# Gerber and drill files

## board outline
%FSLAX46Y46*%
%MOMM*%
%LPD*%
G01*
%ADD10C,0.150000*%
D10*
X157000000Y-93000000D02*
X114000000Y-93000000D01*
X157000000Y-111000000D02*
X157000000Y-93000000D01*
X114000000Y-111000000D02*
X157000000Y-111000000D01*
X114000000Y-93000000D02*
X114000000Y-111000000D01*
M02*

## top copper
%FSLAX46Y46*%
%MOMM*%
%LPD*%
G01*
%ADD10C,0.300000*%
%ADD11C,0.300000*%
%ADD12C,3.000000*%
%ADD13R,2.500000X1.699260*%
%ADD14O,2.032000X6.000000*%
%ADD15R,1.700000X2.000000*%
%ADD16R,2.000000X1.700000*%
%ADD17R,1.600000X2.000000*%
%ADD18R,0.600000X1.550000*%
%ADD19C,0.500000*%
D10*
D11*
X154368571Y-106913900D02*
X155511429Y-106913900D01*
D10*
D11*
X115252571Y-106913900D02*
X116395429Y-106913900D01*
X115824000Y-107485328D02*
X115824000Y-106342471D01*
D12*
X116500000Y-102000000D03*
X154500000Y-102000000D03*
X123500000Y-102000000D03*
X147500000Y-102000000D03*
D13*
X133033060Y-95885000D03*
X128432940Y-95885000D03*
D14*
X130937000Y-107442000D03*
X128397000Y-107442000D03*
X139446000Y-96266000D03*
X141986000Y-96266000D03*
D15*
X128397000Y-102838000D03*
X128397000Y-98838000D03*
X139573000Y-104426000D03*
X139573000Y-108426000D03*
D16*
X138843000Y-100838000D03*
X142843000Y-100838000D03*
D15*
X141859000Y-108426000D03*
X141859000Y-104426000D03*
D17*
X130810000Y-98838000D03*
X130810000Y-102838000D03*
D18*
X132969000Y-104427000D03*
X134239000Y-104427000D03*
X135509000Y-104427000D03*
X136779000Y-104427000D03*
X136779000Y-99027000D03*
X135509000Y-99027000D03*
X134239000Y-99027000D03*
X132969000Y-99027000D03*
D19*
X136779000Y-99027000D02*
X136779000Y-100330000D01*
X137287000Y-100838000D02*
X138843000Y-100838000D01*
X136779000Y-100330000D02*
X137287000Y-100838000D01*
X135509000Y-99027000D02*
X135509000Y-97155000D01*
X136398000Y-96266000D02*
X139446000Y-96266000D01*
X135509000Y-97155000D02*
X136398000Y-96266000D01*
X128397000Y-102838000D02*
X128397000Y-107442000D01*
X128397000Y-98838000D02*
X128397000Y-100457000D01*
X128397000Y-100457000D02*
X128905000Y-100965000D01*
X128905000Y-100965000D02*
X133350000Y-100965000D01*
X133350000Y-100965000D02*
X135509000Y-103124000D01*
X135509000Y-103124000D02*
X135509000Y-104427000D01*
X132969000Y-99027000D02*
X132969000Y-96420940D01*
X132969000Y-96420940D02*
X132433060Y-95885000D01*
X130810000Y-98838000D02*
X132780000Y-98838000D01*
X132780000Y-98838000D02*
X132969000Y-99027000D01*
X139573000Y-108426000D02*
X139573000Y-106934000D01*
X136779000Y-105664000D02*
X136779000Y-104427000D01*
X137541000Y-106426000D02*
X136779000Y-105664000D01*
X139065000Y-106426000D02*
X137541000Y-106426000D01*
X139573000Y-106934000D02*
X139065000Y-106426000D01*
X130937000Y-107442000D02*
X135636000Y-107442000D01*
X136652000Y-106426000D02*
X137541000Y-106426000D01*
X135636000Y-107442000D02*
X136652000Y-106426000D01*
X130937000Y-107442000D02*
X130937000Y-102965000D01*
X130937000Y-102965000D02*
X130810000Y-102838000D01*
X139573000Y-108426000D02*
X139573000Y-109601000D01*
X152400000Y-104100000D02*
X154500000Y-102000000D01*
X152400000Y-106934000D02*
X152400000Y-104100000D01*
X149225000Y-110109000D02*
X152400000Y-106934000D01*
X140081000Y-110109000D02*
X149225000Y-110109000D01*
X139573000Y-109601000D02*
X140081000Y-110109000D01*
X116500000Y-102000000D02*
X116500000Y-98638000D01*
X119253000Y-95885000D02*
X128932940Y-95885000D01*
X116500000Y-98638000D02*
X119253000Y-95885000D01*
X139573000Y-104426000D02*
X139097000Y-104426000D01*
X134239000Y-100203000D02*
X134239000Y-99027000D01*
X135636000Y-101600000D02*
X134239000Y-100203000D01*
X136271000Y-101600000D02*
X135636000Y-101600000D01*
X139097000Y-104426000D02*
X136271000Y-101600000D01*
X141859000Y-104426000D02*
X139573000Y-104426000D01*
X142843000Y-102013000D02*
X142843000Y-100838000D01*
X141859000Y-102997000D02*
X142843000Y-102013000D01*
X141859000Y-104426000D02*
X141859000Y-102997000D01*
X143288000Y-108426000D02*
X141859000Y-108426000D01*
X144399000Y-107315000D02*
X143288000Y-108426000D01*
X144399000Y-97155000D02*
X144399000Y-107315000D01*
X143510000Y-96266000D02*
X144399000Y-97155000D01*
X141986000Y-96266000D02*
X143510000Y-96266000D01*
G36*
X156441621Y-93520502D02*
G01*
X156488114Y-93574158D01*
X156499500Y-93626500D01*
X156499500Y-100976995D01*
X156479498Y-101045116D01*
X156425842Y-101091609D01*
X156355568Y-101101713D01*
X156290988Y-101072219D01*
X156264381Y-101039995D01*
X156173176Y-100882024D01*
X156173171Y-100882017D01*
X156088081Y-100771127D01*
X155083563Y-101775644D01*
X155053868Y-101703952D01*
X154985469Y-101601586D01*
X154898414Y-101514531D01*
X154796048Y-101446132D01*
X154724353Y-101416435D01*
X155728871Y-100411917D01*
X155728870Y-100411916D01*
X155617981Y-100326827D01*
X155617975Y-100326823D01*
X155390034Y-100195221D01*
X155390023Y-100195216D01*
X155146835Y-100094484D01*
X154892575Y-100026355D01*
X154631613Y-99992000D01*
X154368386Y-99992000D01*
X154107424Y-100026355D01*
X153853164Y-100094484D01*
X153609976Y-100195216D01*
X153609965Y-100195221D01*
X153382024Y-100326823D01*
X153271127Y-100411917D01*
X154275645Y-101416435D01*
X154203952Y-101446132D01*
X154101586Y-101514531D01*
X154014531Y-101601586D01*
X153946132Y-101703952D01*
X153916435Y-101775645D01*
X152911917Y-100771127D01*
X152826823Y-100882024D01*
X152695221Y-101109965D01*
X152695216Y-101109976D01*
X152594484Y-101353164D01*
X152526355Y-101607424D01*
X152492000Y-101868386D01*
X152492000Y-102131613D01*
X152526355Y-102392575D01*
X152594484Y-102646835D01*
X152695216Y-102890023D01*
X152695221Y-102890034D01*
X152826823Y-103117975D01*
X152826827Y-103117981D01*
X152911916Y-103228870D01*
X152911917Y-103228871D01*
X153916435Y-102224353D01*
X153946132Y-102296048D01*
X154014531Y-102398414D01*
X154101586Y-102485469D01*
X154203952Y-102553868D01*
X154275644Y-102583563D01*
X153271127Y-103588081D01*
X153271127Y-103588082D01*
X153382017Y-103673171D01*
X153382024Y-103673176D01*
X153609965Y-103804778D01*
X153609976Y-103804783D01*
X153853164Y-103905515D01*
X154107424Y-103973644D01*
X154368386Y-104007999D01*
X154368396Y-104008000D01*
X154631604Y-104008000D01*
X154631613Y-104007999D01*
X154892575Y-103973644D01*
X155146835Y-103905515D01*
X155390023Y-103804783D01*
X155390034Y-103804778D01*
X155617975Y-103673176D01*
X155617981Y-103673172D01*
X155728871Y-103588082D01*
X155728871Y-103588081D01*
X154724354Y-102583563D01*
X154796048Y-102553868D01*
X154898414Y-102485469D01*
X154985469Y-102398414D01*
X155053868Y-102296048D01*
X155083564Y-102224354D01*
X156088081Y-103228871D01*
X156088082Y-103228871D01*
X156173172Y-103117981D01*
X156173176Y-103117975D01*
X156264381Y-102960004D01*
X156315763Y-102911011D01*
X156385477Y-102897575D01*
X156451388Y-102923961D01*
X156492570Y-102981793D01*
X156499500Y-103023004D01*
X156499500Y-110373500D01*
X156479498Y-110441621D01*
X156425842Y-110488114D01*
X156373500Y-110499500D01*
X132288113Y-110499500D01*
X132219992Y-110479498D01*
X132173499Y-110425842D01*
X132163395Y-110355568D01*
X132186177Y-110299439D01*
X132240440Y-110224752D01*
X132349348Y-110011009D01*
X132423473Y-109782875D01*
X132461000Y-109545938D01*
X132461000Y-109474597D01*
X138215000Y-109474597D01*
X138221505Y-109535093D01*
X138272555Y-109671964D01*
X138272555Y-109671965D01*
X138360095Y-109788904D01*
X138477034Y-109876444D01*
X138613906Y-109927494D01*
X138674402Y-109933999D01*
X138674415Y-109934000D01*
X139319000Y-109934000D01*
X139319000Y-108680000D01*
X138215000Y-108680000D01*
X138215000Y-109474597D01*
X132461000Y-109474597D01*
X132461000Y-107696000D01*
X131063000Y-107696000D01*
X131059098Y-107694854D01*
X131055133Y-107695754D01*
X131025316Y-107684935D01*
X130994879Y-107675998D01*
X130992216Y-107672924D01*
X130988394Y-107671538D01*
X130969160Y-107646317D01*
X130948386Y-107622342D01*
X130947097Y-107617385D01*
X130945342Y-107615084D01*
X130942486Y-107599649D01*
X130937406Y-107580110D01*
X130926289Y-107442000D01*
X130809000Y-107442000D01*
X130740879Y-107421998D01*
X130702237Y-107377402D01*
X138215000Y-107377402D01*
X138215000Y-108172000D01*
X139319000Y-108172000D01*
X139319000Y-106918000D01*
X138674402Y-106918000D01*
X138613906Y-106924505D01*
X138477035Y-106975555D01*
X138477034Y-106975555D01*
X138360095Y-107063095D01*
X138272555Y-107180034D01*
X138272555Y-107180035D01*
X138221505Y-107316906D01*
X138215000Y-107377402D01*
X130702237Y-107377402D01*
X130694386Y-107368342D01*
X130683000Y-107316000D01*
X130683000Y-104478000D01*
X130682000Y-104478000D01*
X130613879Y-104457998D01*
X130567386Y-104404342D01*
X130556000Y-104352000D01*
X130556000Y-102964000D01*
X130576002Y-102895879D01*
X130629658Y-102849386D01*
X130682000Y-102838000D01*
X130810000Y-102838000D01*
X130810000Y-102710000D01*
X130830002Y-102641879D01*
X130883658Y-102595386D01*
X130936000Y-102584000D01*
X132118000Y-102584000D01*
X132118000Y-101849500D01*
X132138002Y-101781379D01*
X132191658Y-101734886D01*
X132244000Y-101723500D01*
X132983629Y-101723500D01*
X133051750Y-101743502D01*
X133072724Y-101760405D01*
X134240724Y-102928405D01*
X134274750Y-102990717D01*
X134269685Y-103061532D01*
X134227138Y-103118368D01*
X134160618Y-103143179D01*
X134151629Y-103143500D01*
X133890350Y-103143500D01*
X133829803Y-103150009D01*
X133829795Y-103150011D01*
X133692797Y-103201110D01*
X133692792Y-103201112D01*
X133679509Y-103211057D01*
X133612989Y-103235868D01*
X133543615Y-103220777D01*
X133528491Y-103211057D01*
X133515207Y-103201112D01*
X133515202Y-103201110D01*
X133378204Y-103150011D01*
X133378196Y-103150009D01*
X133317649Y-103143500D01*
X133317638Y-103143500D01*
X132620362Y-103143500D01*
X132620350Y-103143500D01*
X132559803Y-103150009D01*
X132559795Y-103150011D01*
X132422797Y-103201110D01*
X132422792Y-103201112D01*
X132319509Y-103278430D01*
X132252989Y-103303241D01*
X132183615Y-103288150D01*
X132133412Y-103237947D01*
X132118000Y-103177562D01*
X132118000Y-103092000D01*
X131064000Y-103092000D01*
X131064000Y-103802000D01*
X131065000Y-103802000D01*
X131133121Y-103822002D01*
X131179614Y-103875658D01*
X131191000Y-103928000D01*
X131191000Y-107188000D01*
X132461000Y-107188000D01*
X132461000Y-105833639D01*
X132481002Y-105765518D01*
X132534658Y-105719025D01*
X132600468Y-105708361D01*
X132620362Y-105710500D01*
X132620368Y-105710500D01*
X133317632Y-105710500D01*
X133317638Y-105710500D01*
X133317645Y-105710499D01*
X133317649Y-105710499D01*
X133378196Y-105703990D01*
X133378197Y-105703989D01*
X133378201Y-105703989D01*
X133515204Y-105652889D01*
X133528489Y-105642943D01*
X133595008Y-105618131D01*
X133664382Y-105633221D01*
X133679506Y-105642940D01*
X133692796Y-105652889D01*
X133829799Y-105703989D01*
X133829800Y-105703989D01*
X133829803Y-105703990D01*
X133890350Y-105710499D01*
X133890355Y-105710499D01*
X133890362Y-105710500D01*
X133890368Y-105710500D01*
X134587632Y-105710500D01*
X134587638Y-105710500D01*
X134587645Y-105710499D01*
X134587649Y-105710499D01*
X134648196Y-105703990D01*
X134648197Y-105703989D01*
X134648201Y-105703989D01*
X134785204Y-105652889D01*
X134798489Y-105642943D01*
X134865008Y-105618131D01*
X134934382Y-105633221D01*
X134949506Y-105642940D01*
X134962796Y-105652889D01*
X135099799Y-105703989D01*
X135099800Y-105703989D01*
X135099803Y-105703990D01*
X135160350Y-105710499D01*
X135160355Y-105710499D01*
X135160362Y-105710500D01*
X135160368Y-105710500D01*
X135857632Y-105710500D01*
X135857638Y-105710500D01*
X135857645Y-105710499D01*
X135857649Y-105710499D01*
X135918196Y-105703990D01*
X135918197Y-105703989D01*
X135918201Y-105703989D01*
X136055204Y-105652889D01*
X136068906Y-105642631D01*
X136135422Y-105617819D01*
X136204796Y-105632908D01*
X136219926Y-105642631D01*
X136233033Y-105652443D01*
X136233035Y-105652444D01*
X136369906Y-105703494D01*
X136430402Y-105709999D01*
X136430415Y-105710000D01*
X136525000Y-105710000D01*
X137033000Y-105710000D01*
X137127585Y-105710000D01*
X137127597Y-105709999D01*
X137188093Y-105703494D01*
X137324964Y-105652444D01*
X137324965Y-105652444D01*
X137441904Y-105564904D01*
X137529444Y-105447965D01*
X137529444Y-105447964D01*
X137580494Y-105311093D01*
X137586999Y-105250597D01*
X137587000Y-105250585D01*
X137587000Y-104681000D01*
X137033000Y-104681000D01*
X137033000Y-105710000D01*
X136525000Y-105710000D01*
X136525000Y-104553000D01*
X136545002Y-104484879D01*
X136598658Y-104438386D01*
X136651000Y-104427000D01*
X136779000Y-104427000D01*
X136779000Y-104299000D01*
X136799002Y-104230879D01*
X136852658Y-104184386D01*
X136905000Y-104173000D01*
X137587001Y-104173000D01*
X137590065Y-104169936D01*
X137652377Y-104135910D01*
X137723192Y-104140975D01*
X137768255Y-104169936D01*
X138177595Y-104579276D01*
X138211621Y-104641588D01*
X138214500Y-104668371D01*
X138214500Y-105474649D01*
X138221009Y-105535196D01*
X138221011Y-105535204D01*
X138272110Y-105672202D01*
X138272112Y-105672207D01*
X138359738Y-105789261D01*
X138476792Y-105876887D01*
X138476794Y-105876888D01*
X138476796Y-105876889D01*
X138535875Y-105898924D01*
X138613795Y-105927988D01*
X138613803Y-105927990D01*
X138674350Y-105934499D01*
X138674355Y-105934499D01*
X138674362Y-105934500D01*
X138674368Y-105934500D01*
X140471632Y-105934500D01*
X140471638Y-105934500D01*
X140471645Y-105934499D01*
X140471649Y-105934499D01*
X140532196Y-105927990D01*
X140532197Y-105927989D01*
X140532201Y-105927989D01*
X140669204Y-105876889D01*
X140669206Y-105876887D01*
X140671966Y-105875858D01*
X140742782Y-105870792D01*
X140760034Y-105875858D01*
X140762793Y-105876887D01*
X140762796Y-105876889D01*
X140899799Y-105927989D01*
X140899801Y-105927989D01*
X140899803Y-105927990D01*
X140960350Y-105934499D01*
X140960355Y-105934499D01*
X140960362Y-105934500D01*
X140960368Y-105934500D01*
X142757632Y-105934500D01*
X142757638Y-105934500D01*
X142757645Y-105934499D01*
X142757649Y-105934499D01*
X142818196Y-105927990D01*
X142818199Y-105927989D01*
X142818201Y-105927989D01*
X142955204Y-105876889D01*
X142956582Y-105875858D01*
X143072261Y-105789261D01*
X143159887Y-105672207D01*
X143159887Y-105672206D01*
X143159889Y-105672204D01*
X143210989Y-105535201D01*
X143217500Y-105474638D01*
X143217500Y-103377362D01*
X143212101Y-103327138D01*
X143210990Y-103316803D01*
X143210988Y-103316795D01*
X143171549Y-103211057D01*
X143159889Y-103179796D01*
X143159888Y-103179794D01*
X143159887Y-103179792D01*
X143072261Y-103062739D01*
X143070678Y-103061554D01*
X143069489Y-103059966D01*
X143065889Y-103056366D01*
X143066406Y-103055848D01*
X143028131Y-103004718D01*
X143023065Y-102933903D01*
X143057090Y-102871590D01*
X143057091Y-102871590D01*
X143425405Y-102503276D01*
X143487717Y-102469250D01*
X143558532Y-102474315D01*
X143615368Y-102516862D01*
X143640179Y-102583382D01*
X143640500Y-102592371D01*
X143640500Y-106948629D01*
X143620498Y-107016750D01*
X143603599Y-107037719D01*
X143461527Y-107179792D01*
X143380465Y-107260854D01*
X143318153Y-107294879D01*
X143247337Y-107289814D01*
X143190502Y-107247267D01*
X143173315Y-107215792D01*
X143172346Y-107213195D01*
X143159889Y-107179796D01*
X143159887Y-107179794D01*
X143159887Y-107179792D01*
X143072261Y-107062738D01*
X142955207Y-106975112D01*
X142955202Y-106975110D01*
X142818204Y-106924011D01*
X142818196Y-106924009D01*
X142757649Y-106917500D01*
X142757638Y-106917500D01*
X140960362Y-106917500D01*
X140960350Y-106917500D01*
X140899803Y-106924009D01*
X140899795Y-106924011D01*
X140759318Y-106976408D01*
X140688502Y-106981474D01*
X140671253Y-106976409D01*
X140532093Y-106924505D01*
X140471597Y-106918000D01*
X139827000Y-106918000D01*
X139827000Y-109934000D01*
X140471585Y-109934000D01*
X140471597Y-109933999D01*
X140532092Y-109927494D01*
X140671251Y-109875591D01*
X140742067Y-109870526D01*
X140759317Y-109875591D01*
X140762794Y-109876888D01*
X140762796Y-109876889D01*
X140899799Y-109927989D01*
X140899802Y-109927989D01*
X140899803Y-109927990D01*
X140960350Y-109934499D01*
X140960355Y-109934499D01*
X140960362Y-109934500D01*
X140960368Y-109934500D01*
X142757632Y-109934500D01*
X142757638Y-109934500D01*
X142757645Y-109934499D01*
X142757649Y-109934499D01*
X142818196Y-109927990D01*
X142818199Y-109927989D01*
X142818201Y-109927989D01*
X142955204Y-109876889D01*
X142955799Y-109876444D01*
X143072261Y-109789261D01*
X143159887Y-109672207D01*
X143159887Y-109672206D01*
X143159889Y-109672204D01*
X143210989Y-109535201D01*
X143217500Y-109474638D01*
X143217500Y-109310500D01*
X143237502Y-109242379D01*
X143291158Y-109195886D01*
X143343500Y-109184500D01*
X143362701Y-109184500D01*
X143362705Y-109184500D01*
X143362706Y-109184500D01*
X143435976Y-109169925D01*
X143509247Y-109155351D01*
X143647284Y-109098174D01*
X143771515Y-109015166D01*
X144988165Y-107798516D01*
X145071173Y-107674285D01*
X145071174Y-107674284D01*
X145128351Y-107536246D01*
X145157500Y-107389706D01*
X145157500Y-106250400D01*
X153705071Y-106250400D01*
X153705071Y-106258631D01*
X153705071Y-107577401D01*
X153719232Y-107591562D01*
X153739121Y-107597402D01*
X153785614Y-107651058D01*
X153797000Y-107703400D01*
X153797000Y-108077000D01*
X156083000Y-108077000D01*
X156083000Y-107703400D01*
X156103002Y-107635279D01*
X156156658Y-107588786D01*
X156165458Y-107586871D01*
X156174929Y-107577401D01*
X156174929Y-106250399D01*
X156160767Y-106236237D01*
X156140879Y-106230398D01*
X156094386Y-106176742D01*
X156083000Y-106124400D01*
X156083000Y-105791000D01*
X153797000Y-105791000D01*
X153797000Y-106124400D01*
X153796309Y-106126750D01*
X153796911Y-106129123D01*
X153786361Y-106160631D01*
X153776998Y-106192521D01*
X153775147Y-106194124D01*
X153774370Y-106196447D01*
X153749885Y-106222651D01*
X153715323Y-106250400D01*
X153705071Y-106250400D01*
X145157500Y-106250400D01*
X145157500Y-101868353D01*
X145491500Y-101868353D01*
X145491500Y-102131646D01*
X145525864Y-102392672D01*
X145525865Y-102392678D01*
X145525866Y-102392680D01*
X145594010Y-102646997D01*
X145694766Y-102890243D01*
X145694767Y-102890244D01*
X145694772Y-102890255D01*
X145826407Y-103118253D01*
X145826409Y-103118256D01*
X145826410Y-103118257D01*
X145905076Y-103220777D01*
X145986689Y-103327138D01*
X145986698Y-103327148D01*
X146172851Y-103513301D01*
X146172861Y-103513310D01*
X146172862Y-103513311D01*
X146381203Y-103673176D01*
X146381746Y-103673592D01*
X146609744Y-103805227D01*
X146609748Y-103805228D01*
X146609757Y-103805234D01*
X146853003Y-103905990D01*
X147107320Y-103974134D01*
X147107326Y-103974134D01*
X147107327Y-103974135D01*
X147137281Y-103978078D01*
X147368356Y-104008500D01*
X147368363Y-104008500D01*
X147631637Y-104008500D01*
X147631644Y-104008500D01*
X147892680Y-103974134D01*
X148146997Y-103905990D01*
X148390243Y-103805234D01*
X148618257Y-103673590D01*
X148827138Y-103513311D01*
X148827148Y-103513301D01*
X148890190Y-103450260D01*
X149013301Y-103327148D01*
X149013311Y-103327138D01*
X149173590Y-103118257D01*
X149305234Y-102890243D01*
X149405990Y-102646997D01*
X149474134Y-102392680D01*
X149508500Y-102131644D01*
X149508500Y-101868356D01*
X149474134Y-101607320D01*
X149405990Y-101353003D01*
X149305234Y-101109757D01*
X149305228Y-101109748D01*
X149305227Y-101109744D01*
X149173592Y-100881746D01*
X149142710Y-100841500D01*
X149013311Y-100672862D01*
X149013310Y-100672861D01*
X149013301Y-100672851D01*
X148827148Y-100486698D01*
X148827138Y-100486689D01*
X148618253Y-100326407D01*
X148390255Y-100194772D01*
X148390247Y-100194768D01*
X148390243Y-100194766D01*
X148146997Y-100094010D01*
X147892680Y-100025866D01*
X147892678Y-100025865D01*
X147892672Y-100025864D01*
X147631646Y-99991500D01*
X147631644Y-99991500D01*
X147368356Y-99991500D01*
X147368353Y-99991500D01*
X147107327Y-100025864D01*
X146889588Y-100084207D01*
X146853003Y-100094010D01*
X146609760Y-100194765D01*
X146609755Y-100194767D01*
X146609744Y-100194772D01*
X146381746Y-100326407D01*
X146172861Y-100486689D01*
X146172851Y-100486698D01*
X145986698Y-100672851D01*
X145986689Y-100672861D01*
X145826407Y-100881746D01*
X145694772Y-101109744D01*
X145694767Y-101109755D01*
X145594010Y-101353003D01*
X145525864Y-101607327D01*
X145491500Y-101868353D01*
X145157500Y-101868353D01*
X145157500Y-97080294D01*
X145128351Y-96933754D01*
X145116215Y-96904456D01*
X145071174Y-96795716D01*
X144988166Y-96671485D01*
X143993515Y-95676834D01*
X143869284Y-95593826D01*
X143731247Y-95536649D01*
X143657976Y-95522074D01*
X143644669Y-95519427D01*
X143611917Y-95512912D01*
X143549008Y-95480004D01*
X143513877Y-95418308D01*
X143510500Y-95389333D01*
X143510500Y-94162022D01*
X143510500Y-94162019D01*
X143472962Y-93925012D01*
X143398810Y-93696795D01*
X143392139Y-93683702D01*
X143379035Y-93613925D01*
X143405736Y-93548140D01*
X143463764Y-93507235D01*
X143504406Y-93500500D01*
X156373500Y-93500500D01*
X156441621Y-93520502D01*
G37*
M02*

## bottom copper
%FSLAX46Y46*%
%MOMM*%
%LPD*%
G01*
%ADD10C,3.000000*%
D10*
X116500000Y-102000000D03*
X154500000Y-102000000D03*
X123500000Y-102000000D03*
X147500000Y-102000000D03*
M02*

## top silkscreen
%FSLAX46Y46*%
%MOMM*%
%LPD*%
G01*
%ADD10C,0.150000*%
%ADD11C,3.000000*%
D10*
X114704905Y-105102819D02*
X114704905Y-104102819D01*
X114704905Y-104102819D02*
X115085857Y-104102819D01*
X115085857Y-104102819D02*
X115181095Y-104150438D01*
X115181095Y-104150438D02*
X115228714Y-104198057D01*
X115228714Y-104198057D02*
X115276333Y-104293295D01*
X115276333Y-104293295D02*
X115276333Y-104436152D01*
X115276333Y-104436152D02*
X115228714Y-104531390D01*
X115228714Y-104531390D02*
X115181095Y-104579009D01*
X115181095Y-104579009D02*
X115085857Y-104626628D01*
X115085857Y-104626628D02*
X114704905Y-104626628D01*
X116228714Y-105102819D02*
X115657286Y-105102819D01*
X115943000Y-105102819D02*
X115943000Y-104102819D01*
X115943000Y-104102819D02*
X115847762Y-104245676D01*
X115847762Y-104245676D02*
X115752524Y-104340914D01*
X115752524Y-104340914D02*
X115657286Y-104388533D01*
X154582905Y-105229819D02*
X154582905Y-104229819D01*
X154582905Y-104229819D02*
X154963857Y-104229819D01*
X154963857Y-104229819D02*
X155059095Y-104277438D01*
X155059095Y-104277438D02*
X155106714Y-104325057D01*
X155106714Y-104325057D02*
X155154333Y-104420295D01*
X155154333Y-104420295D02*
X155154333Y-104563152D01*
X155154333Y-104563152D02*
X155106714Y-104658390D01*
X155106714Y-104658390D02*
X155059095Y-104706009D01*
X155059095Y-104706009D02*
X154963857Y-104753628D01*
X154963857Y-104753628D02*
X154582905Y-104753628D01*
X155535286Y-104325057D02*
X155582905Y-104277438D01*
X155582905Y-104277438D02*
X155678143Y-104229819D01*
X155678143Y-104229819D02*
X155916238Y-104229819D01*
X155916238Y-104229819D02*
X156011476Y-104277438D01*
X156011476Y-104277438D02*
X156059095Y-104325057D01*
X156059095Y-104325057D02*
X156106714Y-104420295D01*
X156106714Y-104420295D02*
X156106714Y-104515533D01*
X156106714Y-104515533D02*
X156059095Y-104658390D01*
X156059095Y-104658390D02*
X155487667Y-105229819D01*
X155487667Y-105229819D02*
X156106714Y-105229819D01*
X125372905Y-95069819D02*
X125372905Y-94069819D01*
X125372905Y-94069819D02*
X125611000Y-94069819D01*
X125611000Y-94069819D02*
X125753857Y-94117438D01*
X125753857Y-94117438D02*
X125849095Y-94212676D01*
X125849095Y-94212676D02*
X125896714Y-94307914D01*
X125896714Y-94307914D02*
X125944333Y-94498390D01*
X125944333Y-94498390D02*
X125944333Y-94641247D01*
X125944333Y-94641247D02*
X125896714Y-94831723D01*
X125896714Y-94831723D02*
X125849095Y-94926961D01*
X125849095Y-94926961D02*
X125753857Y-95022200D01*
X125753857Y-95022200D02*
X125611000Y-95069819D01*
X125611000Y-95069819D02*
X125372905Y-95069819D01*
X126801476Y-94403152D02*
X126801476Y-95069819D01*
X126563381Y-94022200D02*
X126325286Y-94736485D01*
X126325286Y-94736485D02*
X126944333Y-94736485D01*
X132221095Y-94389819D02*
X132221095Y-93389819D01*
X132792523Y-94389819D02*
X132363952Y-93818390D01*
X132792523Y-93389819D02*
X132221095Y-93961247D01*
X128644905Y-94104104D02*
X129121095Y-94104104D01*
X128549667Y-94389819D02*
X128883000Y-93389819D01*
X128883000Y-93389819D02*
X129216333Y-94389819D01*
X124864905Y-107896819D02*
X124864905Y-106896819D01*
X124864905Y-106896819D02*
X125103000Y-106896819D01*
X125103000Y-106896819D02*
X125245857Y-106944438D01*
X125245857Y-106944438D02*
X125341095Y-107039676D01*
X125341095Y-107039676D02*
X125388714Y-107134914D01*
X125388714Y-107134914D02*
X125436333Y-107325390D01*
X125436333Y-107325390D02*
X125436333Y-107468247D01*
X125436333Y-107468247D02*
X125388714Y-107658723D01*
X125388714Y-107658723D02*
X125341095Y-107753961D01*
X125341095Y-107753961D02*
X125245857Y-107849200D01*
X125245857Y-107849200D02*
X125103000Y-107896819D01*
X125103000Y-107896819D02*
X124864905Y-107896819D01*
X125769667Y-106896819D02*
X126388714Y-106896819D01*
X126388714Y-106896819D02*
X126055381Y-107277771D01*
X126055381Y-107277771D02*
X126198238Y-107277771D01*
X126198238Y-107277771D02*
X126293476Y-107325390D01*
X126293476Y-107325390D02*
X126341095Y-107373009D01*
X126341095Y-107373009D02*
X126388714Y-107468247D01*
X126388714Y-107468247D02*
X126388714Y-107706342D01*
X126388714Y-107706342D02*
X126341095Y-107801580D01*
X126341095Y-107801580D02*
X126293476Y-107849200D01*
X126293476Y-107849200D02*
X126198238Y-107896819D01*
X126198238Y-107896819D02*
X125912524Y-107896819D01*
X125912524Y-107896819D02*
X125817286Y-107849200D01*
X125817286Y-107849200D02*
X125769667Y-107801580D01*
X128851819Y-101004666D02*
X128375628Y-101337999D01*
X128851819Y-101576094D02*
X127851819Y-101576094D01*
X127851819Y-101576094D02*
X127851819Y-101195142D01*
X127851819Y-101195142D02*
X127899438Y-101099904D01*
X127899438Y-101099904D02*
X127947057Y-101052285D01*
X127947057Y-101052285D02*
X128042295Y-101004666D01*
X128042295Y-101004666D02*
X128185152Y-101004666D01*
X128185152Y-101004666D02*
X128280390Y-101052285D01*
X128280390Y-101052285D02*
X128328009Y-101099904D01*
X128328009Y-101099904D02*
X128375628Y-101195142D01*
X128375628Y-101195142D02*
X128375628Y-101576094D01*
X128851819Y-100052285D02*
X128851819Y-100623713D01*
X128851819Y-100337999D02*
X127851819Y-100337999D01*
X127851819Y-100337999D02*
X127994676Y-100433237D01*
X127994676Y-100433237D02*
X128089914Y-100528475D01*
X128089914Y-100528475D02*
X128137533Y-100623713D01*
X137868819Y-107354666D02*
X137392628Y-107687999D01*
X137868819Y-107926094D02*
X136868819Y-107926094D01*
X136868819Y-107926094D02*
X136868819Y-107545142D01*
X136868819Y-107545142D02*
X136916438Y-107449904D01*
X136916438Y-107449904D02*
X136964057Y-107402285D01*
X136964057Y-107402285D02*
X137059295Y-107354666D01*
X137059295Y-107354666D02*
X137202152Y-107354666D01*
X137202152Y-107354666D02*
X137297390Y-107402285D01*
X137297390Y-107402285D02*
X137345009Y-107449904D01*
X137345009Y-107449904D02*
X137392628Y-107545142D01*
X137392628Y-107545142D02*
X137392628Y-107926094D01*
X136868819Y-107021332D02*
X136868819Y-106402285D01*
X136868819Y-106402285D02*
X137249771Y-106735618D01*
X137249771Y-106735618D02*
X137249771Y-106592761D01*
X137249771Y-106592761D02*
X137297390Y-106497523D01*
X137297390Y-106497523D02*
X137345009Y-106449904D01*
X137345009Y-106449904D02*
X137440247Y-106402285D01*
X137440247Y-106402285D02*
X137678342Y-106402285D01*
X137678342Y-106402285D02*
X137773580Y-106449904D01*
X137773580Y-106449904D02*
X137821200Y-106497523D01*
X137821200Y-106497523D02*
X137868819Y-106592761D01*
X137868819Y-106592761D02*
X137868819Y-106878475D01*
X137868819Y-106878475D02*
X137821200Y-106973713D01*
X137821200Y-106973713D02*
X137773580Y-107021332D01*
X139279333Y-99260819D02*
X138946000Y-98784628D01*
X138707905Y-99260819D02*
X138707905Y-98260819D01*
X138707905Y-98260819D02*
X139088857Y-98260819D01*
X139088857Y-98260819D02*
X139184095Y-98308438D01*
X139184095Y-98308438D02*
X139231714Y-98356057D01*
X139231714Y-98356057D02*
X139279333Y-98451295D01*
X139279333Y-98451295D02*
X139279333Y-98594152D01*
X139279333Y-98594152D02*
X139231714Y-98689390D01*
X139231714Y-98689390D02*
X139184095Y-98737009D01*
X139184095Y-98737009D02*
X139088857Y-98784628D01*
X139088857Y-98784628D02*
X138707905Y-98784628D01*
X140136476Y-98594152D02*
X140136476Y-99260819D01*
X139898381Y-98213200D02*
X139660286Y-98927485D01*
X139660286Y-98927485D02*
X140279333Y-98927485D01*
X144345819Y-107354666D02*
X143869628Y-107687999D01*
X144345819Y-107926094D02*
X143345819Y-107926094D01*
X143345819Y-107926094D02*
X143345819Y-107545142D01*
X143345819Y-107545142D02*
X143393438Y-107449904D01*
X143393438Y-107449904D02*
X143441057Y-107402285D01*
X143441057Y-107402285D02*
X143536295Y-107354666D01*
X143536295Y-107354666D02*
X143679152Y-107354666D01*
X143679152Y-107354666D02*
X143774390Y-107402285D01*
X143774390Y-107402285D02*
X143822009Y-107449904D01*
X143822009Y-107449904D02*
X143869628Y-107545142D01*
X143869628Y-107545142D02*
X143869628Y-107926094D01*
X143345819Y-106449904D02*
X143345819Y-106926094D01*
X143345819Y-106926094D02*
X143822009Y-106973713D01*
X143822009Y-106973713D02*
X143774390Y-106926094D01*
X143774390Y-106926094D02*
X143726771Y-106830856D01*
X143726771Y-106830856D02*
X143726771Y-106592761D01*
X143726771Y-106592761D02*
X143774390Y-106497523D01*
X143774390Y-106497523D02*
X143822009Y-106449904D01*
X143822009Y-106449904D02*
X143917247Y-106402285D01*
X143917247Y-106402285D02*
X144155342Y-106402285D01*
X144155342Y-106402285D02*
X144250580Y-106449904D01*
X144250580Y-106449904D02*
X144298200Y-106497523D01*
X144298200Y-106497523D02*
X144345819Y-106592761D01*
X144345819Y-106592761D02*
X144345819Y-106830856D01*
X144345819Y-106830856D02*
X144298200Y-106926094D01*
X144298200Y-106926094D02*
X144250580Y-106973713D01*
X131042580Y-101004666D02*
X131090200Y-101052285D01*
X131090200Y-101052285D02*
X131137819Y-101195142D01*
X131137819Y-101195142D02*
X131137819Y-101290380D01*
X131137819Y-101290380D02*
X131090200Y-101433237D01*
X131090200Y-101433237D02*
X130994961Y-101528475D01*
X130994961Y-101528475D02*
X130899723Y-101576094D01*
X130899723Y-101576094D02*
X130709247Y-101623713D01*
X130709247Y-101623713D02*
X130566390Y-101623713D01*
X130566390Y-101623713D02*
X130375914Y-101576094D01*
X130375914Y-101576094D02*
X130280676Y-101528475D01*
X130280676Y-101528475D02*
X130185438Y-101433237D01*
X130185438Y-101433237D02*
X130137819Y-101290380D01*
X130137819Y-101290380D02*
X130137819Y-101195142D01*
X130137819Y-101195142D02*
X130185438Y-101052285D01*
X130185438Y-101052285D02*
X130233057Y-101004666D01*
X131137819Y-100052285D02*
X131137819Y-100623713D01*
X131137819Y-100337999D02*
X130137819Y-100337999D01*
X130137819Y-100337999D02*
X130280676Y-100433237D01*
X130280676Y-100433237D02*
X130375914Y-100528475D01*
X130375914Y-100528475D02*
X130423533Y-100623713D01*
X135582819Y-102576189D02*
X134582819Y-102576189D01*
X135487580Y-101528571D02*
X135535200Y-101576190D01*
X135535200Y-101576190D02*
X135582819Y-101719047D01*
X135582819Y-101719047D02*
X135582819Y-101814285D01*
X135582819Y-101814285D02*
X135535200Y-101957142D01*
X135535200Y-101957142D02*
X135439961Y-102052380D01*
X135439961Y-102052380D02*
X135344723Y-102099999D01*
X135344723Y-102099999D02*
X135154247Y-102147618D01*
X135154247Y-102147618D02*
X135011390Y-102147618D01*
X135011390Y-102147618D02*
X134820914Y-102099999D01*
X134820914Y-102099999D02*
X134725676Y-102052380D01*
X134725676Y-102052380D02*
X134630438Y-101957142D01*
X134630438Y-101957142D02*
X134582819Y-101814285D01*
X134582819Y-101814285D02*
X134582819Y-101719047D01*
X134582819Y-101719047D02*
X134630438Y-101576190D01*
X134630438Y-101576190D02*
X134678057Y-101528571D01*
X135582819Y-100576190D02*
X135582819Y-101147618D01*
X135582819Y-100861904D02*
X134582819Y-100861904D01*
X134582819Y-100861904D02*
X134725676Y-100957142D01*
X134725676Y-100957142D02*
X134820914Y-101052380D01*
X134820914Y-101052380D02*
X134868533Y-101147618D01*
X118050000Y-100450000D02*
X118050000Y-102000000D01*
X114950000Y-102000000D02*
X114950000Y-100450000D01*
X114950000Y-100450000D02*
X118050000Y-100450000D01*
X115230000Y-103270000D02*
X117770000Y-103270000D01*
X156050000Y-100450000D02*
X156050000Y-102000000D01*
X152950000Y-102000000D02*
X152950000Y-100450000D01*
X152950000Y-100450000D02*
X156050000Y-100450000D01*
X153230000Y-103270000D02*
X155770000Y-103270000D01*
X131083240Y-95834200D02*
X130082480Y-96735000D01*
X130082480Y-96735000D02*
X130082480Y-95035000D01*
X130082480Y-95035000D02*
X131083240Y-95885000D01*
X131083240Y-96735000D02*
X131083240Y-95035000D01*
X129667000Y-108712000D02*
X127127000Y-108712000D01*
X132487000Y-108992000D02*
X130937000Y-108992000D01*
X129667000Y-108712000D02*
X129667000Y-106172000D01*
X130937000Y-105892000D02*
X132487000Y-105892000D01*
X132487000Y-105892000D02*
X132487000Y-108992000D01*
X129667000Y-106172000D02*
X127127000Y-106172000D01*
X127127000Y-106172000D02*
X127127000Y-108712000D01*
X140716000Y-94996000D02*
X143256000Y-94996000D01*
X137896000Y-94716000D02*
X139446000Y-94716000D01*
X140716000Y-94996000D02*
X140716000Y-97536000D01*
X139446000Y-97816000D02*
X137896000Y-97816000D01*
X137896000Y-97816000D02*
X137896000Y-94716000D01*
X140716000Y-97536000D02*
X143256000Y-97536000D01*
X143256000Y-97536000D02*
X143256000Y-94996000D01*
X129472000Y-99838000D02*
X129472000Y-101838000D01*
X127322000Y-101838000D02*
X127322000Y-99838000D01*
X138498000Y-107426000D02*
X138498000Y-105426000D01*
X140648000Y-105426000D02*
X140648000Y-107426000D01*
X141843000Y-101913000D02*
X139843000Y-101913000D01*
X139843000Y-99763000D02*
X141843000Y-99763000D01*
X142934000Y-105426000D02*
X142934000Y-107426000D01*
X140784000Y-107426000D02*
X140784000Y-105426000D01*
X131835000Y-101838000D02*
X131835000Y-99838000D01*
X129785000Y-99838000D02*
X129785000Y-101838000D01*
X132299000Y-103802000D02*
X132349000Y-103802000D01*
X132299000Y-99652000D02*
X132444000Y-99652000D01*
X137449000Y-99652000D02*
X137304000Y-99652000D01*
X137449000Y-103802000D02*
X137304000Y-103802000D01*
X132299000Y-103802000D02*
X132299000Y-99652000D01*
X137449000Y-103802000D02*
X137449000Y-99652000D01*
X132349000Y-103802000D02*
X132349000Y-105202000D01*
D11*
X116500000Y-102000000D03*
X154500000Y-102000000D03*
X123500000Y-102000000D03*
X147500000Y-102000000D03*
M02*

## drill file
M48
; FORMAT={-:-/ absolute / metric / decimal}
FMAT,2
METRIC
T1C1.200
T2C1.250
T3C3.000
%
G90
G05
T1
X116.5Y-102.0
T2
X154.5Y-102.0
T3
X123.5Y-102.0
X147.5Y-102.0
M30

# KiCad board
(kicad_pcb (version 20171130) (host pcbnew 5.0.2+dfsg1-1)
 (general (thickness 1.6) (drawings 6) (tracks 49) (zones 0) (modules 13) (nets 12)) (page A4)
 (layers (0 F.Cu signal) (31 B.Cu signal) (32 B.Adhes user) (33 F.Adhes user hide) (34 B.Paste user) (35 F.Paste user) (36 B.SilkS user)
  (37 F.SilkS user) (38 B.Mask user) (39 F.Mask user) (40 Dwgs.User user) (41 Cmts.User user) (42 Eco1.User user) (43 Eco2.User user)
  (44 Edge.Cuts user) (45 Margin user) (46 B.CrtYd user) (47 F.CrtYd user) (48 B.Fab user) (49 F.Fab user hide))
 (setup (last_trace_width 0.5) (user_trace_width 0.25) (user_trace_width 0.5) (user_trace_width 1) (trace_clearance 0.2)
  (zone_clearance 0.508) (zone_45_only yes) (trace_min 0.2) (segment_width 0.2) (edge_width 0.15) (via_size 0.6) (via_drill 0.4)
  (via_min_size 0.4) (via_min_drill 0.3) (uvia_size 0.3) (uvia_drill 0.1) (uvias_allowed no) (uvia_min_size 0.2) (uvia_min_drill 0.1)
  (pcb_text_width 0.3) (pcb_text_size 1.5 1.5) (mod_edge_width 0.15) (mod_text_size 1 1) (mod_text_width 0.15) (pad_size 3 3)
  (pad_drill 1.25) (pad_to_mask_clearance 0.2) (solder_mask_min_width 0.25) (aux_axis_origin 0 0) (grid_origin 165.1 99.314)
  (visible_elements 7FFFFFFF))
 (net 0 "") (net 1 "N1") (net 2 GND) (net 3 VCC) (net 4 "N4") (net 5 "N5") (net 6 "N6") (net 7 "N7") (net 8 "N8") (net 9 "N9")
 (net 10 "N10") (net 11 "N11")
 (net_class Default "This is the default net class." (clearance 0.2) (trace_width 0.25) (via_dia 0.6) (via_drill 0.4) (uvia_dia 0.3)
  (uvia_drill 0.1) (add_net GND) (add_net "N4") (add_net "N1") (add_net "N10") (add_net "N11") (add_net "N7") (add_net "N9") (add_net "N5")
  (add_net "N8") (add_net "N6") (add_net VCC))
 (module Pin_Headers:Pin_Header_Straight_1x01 (layer F.Cu) (at 116.5 102)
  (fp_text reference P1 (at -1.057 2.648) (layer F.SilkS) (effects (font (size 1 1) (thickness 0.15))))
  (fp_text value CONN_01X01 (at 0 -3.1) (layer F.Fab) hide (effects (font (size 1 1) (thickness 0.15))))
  (fp_line (start 1.55 -1.55) (end 1.55 0) (layer F.SilkS) (width 0.15))
  (fp_line (start -1.55 0) (end -1.55 -1.55) (layer F.SilkS) (width 0.15))
  (fp_line (start -1.55 -1.55) (end 1.55 -1.55) (layer F.SilkS) (width 0.15))
  (fp_line (start -1.27 1.27) (end 1.27 1.27) (layer F.SilkS) (width 0.15))
  (pad 1 thru_hole circle (at 0 0) (size 3 3) (drill 1.2) (layers F.Cu F.SilkS F.Mask) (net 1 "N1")))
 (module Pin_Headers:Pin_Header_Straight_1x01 (layer F.Cu) (at 154.5 102)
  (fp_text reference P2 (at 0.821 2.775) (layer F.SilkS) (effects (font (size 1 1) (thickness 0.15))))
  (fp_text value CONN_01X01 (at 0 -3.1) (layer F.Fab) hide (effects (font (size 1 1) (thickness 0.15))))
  (fp_line (start 1.55 -1.55) (end 1.55 0) (layer F.SilkS) (width 0.15))
  (fp_line (start -1.55 0) (end -1.55 -1.55) (layer F.SilkS) (width 0.15))
  (fp_line (start -1.55 -1.55) (end 1.55 -1.55) (layer F.SilkS) (width 0.15))
  (fp_line (start -1.27 1.27) (end 1.27 1.27) (layer F.SilkS) (width 0.15))
  (pad 1 thru_hole circle (at 0 0) (size 3 3) (drill 1.25) (layers *.Mask F.Cu F.SilkS) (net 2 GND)))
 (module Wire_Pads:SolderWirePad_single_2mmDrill (layer F.Cu) (at 123.5 102)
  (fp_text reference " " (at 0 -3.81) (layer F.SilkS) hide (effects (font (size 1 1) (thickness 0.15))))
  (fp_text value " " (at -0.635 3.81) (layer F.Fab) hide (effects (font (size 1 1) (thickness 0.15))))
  (pad 1 thru_hole circle (at 0 0) (size 3 3) (drill 3) (layers *.Mask F.Cu F.SilkS)))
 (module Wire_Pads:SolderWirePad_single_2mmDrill (layer F.Cu) (at 147.5 102)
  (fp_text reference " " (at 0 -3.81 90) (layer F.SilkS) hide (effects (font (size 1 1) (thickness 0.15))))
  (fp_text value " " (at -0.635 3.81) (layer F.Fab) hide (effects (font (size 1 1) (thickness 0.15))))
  (pad 1 thru_hole circle (at 0 0) (size 3 3) (drill 3) (layers *.Mask F.Cu F.SilkS)))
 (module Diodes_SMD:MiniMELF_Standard (layer F.Cu) (at 130.683 95.885 180)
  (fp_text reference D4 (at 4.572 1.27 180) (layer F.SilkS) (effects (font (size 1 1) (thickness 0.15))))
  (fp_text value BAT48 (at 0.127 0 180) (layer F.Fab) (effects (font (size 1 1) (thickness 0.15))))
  (fp_line (start -0.40024 0.0508) (end 0.60052 -0.85) (layer F.SilkS) (width 0.15))
  (fp_line (start 0.60052 -0.85) (end 0.60052 0.85) (layer F.SilkS) (width 0.15))
  (fp_line (start 0.60052 0.85) (end -0.40024 0) (layer F.SilkS) (width 0.15))
  (fp_line (start -0.40024 -0.85) (end -0.40024 0.85) (layer F.SilkS) (width 0.15))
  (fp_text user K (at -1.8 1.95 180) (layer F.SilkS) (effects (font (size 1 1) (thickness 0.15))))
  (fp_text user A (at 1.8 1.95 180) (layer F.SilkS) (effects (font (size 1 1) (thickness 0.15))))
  (pad 1 smd rect (at -1.75006 0 180) (size 2.5 1.69926) (drill (offset -0.6 0)) (layers F.Cu F.Paste F.Mask) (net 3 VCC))
  (pad 2 smd rect (at 1.75006 0 180) (size 2.5 1.69926) (drill (offset 0.5 0)) (layers F.Cu F.Paste F.Mask) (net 1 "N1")))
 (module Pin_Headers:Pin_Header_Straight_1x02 (layer F.Cu) (at 130.937 107.442 270)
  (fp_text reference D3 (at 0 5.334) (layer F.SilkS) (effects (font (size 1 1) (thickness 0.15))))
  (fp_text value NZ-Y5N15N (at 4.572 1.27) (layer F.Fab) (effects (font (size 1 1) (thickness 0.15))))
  (fp_line (start 1.27 1.27) (end 1.27 3.81) (layer F.SilkS) (width 0.15))
  (fp_line (start 1.55 -1.55) (end 1.55 0) (layer F.SilkS) (width 0.15))
  (fp_line (start 1.27 1.27) (end -1.27 1.27) (layer F.SilkS) (width 0.15))
  (fp_line (start -1.55 0) (end -1.55 -1.55) (layer F.SilkS) (width 0.15))
  (fp_line (start -1.55 -1.55) (end 1.55 -1.55) (layer F.SilkS) (width 0.15))
  (fp_line (start -1.27 1.27) (end -1.27 3.81) (layer F.SilkS) (width 0.15))
  (fp_line (start -1.27 3.81) (end 1.27 3.81) (layer F.SilkS) (width 0.15))
  (pad 1 smd oval (at 0 0 270) (size 6 2.032) (layers F.Cu F.Paste F.Mask) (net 2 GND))
  (pad 2 smd oval (at 0 2.54 270) (size 6 2.032) (layers F.Cu F.Paste F.Mask) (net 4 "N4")))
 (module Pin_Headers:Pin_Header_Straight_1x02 (layer F.Cu) (at 139.446 96.266 90)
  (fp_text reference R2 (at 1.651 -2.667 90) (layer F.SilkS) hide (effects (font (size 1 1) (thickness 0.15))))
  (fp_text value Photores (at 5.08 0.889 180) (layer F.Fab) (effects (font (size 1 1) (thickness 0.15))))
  (fp_line (start 1.27 1.27) (end 1.27 3.81) (layer F.SilkS) (width 0.15))
  (fp_line (start 1.55 -1.55) (end 1.55 0) (layer F.SilkS) (width 0.15))
  (fp_line (start 1.27 1.27) (end -1.27 1.27) (layer F.SilkS) (width 0.15))
  (fp_line (start -1.55 0) (end -1.55 -1.55) (layer F.SilkS) (width 0.15))
  (fp_line (start -1.55 -1.55) (end 1.55 -1.55) (layer F.SilkS) (width 0.15))
  (fp_line (start -1.27 1.27) (end -1.27 3.81) (layer F.SilkS) (width 0.15))
  (fp_line (start -1.27 3.81) (end 1.27 3.81) (layer F.SilkS) (width 0.15))
  (pad 1 smd oval (at 0 0 90) (size 6 2.032) (layers F.Cu F.Paste F.Mask) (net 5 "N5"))
  (pad 2 smd oval (at 0 2.54 90) (size 6 2.032) (layers F.Cu F.Paste F.Mask) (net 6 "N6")))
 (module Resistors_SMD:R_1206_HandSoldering (layer F.Cu) (at 128.397 100.838 90)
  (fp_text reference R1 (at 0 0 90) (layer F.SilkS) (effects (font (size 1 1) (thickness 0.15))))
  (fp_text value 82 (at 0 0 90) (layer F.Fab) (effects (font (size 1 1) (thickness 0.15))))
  (fp_line (start 1 1.075) (end -1 1.075) (layer F.SilkS) (width 0.15))
  (fp_line (start -1 -1.075) (end 1 -1.075) (layer F.SilkS) (width 0.15))
  (pad 1 smd rect (at -2 0 90) (size 2 1.7) (layers F.Cu F.Paste F.Mask) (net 4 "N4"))
  (pad 2 smd rect (at 2 0 90) (size 2 1.7) (layers F.Cu F.Paste F.Mask) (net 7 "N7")))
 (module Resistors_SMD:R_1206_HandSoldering (layer F.Cu) (at 139.573 106.426 270)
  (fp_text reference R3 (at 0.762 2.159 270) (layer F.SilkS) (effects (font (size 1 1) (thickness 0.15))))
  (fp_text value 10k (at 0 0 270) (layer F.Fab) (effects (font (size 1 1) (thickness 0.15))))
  (fp_line (start 1 1.075) (end -1 1.075) (layer F.SilkS) (width 0.15))
  (fp_line (start -1 -1.075) (end 1 -1.075) (layer F.SilkS) (width 0.15))
  (pad 1 smd rect (at -2 0 270) (size 2 1.7) (layers F.Cu F.Paste F.Mask) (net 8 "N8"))
  (pad 2 smd rect (at 2 0 270) (size 2 1.7) (layers F.Cu F.Paste F.Mask) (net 2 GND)))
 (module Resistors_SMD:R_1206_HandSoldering (layer F.Cu) (at 140.843 100.838)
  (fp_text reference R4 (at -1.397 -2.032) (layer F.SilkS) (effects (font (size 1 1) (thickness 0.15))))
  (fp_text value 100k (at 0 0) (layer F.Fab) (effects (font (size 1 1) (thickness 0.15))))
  (fp_line (start 1 1.075) (end -1 1.075) (layer F.SilkS) (width 0.15))
  (fp_line (start -1 -1.075) (end 1 -1.075) (layer F.SilkS) (width 0.15))
  (pad 1 smd rect (at -2 0) (size 2 1.7) (layers F.Cu F.Paste F.Mask) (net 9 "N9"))
  (pad 2 smd rect (at 2 0) (size 2 1.7) (layers F.Cu F.Paste F.Mask) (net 8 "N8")))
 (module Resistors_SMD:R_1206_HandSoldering (layer F.Cu) (at 141.859 106.426 90)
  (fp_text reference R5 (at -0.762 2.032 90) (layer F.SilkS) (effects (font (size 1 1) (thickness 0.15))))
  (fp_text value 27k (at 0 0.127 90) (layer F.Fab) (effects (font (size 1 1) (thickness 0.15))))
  (fp_line (start 1 1.075) (end -1 1.075) (layer F.SilkS) (width 0.15))
  (fp_line (start -1 -1.075) (end 1 -1.075) (layer F.SilkS) (width 0.15))
  (pad 1 smd rect (at -2 0 90) (size 2 1.7) (layers F.Cu F.Paste F.Mask) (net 6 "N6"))
  (pad 2 smd rect (at 2 0 90) (size 2 1.7) (layers F.Cu F.Paste F.Mask) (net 8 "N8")))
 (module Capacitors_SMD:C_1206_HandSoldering (layer F.Cu) (at 130.81 100.838 270)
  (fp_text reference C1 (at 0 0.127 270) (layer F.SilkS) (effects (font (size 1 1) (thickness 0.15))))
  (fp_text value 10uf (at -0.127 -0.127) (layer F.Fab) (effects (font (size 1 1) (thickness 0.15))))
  (fp_line (start 1 -1.025) (end -1 -1.025) (layer F.SilkS) (width 0.15))
  (fp_line (start -1 1.025) (end 1 1.025) (layer F.SilkS) (width 0.15))
  (pad 1 smd rect (at -2 0 270) (size 2 1.6) (layers F.Cu F.Paste F.Mask) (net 3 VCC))
  (pad 2 smd rect (at 2 0 270) (size 2 1.6) (layers F.Cu F.Paste F.Mask) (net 2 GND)))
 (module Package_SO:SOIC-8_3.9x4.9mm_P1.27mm (layer F.Cu) (at 134.874 101.727 90)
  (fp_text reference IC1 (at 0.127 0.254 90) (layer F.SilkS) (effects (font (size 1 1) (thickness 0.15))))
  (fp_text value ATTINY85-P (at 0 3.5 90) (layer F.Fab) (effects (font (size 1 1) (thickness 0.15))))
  (fp_line (start -2.075 -2.575) (end -2.075 -2.525) (layer F.SilkS) (width 0.15))
  (fp_line (start 2.075 -2.575) (end 2.075 -2.43) (layer F.SilkS) (width 0.15))
  (fp_line (start 2.075 2.575) (end 2.075 2.43) (layer F.SilkS) (width 0.15))
  (fp_line (start -2.075 2.575) (end -2.075 2.43) (layer F.SilkS) (width 0.15))
  (fp_line (start -2.075 -2.575) (end 2.075 -2.575) (layer F.SilkS) (width 0.15))
  (fp_line (start -2.075 2.575) (end 2.075 2.575) (layer F.SilkS) (width 0.15))
  (fp_line (start -2.075 -2.525) (end -3.475 -2.525) (layer F.SilkS) (width 0.15))
  (pad 1 smd rect (at -2.7 -1.905 90) (size 1.55 0.6) (layers F.Cu F.Paste F.Mask) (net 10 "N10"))
  (pad 2 smd rect (at -2.7 -0.635 90) (size 1.55 0.6) (layers F.Cu F.Paste F.Mask) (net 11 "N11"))
  (pad 3 smd rect (at -2.7 0.635 90) (size 1.55 0.6) (layers F.Cu F.Paste F.Mask) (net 7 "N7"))
  (pad 4 smd rect (at -2.7 1.905 90) (size 1.55 0.6) (layers F.Cu F.Paste F.Mask) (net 2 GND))
  (pad 5 smd rect (at 2.7 1.905 90) (size 1.55 0.6) (layers F.Cu F.Paste F.Mask) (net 9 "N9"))
  (pad 6 smd rect (at 2.7 0.635 90) (size 1.55 0.6) (layers F.Cu F.Paste F.Mask) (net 5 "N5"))
  (pad 7 smd rect (at 2.7 -0.635 90) (size 1.55 0.6) (layers F.Cu F.Paste F.Mask) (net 8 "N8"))
  (pad 8 smd rect (at 2.7 -1.905 90) (size 1.55 0.6) (layers F.Cu F.Paste F.Mask) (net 3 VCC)))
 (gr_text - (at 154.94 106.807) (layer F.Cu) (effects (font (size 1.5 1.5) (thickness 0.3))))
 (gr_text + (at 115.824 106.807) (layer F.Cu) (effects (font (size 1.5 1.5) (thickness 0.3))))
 (gr_line (start 157 93) (end 114 93) (angle 90) (layer Edge.Cuts) (width 0.15))
 (gr_line (start 157 111) (end 157 93) (angle 90) (layer Edge.Cuts) (width 0.15))
 (gr_line (start 114 111) (end 157 111) (angle 90) (layer Edge.Cuts) (width 0.15))
 (gr_line (start 114 93) (end 114 111) (angle 90) (layer Edge.Cuts) (width 0.15))
 (segment (start 136.779 99.027) (end 136.779 100.33) (width 0.5) (layer F.Cu) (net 9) (status 400000))
 (segment (start 137.287 100.838) (end 138.843 100.838) (width 0.5) (layer F.Cu) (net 9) (status 800000))
 (segment (start 136.779 100.33) (end 137.287 100.838) (width 0.5) (layer F.Cu) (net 9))
 (segment (start 135.509 99.027) (end 135.509 97.155) (width 0.5) (layer F.Cu) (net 5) (status 400000))
 (segment (start 136.398 96.266) (end 139.446 96.266) (width 0.5) (layer F.Cu) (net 5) (status 800000))
 (segment (start 135.509 97.155) (end 136.398 96.266) (width 0.5) (layer F.Cu) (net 5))
 (segment (start 128.397 102.838) (end 128.397 107.442) (width 0.5) (layer F.Cu) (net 4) (status C00000))
 (segment (start 128.397 98.838) (end 128.397 100.457) (width 0.5) (layer F.Cu) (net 7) (status 400000))
 (segment (start 128.397 100.457) (end 128.905 100.965) (width 0.5) (layer F.Cu) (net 7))
 (segment (start 128.905 100.965) (end 133.35 100.965) (width 0.5) (layer F.Cu) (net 7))
 (segment (start 133.35 100.965) (end 135.509 103.124) (width 0.5) (layer F.Cu) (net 7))
 (segment (start 135.509 103.124) (end 135.509 104.427) (width 0.5) (layer F.Cu) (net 7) (status 800000))
 (segment (start 132.969 99.027) (end 132.969 96.42094) (width 0.5) (layer F.Cu) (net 3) (status C00000))
 (segment (start 132.969 96.42094) (end 132.43306 95.885) (width 0.5) (layer F.Cu) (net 3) (status C00000))
 (segment (start 130.81 98.838) (end 132.78 98.838) (width 0.5) (layer F.Cu) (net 3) (status C00000))
 (segment (start 132.78 98.838) (end 132.969 99.027) (width 0.5) (layer F.Cu) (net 3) (status C00000))
 (segment (start 139.573 108.426) (end 139.573 106.934) (width 0.5) (layer F.Cu) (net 2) (status 400000))
 (segment (start 136.779 105.664) (end 136.779 104.427) (width 0.5) (layer F.Cu) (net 2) (status 800000))
 (segment (start 137.541 106.426) (end 136.779 105.664) (width 0.5) (layer F.Cu) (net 2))
 (segment (start 139.065 106.426) (end 137.541 106.426) (width 0.5) (layer F.Cu) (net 2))
 (segment (start 139.573 106.934) (end 139.065 106.426) (width 0.5) (layer F.Cu) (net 2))
 (segment (start 130.937 107.442) (end 135.636 107.442) (width 0.5) (layer F.Cu) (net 2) (status 400000))
 (segment (start 136.652 106.426) (end 137.541 106.426) (width 0.5) (layer F.Cu) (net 2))
 (segment (start 135.636 107.442) (end 136.652 106.426) (width 0.5) (layer F.Cu) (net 2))
 (segment (start 130.937 107.442) (end 130.937 102.965) (width 0.5) (layer F.Cu) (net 2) (status C00000))
 (segment (start 130.937 102.965) (end 130.81 102.838) (width 0.5) (layer F.Cu) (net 2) (status C00000))
 (segment (start 139.573 108.426) (end 139.573 109.601) (width 0.5) (layer F.Cu) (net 2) (status 400000))
 (segment (start 152.4 104.1) (end 154.5 102) (width 0.5) (layer F.Cu) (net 2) (status 800000))
 (segment (start 152.4 106.934) (end 152.4 104.1) (width 0.5) (layer F.Cu) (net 2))
 (segment (start 149.225 110.109) (end 152.4 106.934) (width 0.5) (layer F.Cu) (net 2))
 (segment (start 140.081 110.109) (end 149.225 110.109) (width 0.5) (layer F.Cu) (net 2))
 (segment (start 139.573 109.601) (end 140.081 110.109) (width 0.5) (layer F.Cu) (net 2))
 (segment (start 116.5 102) (end 116.5 98.638) (width 0.5) (layer F.Cu) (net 1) (status 400000))
 (segment (start 119.253 95.885) (end 128.93294 95.885) (width 0.5) (layer F.Cu) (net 1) (status 800000))
 (segment (start 116.5 98.638) (end 119.253 95.885) (width 0.5) (layer F.Cu) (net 1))
 (segment (start 139.573 104.426) (end 139.097 104.426) (width 0.5) (layer F.Cu) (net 8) (status C00000))
 (segment (start 134.239 100.203) (end 134.239 99.027) (width 0.5) (layer F.Cu) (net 8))
 (segment (start 135.636 101.6) (end 134.239 100.203) (width 0.5) (layer F.Cu) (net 8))
 (segment (start 136.271 101.6) (end 135.636 101.6) (width 0.5) (layer F.Cu) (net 8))
 (segment (start 139.097 104.426) (end 136.271 101.6) (width 0.5) (layer F.Cu) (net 8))
 (segment (start 141.859 104.426) (end 139.573 104.426) (width 0.5) (layer F.Cu) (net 8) (status C00000))
 (segment (start 142.843 102.013) (end 142.843 100.838) (width 0.5) (layer F.Cu) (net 8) (status 800000))
 (segment (start 141.859 102.997) (end 142.843 102.013) (width 0.5) (layer F.Cu) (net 8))
 (segment (start 141.859 104.426) (end 141.859 102.997) (width 0.5) (layer F.Cu) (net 8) (status 400000))
 (segment (start 143.288 108.426) (end 141.859 108.426) (width 0.5) (layer F.Cu) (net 6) (status 800000))
 (segment (start 144.399 107.315) (end 143.288 108.426) (width 0.5) (layer F.Cu) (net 6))
 (segment (start 144.399 97.155) (end 144.399 107.315) (width 0.5) (layer F.Cu) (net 6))
 (segment (start 143.51 96.266) (end 144.399 97.155) (width 0.5) (layer F.Cu) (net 6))
 (segment (start 141.986 96.266) (end 143.51 96.266) (width 0.5) (layer F.Cu) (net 6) (status 400000))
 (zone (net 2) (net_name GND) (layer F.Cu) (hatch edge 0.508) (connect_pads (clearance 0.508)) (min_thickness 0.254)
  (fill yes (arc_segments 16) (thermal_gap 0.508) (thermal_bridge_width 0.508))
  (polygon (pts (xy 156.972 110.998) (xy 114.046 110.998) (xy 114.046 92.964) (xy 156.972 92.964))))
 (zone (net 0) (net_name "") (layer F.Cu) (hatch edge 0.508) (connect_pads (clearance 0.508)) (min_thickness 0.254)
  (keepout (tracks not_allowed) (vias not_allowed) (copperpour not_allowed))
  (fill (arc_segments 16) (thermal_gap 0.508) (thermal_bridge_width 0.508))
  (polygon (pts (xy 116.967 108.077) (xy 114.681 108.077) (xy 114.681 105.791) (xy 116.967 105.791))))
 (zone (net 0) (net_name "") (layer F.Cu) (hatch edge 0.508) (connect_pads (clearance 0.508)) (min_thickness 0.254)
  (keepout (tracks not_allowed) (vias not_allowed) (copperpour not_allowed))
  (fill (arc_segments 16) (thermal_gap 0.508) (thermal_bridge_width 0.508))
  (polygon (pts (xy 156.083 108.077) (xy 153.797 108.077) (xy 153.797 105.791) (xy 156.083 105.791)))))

